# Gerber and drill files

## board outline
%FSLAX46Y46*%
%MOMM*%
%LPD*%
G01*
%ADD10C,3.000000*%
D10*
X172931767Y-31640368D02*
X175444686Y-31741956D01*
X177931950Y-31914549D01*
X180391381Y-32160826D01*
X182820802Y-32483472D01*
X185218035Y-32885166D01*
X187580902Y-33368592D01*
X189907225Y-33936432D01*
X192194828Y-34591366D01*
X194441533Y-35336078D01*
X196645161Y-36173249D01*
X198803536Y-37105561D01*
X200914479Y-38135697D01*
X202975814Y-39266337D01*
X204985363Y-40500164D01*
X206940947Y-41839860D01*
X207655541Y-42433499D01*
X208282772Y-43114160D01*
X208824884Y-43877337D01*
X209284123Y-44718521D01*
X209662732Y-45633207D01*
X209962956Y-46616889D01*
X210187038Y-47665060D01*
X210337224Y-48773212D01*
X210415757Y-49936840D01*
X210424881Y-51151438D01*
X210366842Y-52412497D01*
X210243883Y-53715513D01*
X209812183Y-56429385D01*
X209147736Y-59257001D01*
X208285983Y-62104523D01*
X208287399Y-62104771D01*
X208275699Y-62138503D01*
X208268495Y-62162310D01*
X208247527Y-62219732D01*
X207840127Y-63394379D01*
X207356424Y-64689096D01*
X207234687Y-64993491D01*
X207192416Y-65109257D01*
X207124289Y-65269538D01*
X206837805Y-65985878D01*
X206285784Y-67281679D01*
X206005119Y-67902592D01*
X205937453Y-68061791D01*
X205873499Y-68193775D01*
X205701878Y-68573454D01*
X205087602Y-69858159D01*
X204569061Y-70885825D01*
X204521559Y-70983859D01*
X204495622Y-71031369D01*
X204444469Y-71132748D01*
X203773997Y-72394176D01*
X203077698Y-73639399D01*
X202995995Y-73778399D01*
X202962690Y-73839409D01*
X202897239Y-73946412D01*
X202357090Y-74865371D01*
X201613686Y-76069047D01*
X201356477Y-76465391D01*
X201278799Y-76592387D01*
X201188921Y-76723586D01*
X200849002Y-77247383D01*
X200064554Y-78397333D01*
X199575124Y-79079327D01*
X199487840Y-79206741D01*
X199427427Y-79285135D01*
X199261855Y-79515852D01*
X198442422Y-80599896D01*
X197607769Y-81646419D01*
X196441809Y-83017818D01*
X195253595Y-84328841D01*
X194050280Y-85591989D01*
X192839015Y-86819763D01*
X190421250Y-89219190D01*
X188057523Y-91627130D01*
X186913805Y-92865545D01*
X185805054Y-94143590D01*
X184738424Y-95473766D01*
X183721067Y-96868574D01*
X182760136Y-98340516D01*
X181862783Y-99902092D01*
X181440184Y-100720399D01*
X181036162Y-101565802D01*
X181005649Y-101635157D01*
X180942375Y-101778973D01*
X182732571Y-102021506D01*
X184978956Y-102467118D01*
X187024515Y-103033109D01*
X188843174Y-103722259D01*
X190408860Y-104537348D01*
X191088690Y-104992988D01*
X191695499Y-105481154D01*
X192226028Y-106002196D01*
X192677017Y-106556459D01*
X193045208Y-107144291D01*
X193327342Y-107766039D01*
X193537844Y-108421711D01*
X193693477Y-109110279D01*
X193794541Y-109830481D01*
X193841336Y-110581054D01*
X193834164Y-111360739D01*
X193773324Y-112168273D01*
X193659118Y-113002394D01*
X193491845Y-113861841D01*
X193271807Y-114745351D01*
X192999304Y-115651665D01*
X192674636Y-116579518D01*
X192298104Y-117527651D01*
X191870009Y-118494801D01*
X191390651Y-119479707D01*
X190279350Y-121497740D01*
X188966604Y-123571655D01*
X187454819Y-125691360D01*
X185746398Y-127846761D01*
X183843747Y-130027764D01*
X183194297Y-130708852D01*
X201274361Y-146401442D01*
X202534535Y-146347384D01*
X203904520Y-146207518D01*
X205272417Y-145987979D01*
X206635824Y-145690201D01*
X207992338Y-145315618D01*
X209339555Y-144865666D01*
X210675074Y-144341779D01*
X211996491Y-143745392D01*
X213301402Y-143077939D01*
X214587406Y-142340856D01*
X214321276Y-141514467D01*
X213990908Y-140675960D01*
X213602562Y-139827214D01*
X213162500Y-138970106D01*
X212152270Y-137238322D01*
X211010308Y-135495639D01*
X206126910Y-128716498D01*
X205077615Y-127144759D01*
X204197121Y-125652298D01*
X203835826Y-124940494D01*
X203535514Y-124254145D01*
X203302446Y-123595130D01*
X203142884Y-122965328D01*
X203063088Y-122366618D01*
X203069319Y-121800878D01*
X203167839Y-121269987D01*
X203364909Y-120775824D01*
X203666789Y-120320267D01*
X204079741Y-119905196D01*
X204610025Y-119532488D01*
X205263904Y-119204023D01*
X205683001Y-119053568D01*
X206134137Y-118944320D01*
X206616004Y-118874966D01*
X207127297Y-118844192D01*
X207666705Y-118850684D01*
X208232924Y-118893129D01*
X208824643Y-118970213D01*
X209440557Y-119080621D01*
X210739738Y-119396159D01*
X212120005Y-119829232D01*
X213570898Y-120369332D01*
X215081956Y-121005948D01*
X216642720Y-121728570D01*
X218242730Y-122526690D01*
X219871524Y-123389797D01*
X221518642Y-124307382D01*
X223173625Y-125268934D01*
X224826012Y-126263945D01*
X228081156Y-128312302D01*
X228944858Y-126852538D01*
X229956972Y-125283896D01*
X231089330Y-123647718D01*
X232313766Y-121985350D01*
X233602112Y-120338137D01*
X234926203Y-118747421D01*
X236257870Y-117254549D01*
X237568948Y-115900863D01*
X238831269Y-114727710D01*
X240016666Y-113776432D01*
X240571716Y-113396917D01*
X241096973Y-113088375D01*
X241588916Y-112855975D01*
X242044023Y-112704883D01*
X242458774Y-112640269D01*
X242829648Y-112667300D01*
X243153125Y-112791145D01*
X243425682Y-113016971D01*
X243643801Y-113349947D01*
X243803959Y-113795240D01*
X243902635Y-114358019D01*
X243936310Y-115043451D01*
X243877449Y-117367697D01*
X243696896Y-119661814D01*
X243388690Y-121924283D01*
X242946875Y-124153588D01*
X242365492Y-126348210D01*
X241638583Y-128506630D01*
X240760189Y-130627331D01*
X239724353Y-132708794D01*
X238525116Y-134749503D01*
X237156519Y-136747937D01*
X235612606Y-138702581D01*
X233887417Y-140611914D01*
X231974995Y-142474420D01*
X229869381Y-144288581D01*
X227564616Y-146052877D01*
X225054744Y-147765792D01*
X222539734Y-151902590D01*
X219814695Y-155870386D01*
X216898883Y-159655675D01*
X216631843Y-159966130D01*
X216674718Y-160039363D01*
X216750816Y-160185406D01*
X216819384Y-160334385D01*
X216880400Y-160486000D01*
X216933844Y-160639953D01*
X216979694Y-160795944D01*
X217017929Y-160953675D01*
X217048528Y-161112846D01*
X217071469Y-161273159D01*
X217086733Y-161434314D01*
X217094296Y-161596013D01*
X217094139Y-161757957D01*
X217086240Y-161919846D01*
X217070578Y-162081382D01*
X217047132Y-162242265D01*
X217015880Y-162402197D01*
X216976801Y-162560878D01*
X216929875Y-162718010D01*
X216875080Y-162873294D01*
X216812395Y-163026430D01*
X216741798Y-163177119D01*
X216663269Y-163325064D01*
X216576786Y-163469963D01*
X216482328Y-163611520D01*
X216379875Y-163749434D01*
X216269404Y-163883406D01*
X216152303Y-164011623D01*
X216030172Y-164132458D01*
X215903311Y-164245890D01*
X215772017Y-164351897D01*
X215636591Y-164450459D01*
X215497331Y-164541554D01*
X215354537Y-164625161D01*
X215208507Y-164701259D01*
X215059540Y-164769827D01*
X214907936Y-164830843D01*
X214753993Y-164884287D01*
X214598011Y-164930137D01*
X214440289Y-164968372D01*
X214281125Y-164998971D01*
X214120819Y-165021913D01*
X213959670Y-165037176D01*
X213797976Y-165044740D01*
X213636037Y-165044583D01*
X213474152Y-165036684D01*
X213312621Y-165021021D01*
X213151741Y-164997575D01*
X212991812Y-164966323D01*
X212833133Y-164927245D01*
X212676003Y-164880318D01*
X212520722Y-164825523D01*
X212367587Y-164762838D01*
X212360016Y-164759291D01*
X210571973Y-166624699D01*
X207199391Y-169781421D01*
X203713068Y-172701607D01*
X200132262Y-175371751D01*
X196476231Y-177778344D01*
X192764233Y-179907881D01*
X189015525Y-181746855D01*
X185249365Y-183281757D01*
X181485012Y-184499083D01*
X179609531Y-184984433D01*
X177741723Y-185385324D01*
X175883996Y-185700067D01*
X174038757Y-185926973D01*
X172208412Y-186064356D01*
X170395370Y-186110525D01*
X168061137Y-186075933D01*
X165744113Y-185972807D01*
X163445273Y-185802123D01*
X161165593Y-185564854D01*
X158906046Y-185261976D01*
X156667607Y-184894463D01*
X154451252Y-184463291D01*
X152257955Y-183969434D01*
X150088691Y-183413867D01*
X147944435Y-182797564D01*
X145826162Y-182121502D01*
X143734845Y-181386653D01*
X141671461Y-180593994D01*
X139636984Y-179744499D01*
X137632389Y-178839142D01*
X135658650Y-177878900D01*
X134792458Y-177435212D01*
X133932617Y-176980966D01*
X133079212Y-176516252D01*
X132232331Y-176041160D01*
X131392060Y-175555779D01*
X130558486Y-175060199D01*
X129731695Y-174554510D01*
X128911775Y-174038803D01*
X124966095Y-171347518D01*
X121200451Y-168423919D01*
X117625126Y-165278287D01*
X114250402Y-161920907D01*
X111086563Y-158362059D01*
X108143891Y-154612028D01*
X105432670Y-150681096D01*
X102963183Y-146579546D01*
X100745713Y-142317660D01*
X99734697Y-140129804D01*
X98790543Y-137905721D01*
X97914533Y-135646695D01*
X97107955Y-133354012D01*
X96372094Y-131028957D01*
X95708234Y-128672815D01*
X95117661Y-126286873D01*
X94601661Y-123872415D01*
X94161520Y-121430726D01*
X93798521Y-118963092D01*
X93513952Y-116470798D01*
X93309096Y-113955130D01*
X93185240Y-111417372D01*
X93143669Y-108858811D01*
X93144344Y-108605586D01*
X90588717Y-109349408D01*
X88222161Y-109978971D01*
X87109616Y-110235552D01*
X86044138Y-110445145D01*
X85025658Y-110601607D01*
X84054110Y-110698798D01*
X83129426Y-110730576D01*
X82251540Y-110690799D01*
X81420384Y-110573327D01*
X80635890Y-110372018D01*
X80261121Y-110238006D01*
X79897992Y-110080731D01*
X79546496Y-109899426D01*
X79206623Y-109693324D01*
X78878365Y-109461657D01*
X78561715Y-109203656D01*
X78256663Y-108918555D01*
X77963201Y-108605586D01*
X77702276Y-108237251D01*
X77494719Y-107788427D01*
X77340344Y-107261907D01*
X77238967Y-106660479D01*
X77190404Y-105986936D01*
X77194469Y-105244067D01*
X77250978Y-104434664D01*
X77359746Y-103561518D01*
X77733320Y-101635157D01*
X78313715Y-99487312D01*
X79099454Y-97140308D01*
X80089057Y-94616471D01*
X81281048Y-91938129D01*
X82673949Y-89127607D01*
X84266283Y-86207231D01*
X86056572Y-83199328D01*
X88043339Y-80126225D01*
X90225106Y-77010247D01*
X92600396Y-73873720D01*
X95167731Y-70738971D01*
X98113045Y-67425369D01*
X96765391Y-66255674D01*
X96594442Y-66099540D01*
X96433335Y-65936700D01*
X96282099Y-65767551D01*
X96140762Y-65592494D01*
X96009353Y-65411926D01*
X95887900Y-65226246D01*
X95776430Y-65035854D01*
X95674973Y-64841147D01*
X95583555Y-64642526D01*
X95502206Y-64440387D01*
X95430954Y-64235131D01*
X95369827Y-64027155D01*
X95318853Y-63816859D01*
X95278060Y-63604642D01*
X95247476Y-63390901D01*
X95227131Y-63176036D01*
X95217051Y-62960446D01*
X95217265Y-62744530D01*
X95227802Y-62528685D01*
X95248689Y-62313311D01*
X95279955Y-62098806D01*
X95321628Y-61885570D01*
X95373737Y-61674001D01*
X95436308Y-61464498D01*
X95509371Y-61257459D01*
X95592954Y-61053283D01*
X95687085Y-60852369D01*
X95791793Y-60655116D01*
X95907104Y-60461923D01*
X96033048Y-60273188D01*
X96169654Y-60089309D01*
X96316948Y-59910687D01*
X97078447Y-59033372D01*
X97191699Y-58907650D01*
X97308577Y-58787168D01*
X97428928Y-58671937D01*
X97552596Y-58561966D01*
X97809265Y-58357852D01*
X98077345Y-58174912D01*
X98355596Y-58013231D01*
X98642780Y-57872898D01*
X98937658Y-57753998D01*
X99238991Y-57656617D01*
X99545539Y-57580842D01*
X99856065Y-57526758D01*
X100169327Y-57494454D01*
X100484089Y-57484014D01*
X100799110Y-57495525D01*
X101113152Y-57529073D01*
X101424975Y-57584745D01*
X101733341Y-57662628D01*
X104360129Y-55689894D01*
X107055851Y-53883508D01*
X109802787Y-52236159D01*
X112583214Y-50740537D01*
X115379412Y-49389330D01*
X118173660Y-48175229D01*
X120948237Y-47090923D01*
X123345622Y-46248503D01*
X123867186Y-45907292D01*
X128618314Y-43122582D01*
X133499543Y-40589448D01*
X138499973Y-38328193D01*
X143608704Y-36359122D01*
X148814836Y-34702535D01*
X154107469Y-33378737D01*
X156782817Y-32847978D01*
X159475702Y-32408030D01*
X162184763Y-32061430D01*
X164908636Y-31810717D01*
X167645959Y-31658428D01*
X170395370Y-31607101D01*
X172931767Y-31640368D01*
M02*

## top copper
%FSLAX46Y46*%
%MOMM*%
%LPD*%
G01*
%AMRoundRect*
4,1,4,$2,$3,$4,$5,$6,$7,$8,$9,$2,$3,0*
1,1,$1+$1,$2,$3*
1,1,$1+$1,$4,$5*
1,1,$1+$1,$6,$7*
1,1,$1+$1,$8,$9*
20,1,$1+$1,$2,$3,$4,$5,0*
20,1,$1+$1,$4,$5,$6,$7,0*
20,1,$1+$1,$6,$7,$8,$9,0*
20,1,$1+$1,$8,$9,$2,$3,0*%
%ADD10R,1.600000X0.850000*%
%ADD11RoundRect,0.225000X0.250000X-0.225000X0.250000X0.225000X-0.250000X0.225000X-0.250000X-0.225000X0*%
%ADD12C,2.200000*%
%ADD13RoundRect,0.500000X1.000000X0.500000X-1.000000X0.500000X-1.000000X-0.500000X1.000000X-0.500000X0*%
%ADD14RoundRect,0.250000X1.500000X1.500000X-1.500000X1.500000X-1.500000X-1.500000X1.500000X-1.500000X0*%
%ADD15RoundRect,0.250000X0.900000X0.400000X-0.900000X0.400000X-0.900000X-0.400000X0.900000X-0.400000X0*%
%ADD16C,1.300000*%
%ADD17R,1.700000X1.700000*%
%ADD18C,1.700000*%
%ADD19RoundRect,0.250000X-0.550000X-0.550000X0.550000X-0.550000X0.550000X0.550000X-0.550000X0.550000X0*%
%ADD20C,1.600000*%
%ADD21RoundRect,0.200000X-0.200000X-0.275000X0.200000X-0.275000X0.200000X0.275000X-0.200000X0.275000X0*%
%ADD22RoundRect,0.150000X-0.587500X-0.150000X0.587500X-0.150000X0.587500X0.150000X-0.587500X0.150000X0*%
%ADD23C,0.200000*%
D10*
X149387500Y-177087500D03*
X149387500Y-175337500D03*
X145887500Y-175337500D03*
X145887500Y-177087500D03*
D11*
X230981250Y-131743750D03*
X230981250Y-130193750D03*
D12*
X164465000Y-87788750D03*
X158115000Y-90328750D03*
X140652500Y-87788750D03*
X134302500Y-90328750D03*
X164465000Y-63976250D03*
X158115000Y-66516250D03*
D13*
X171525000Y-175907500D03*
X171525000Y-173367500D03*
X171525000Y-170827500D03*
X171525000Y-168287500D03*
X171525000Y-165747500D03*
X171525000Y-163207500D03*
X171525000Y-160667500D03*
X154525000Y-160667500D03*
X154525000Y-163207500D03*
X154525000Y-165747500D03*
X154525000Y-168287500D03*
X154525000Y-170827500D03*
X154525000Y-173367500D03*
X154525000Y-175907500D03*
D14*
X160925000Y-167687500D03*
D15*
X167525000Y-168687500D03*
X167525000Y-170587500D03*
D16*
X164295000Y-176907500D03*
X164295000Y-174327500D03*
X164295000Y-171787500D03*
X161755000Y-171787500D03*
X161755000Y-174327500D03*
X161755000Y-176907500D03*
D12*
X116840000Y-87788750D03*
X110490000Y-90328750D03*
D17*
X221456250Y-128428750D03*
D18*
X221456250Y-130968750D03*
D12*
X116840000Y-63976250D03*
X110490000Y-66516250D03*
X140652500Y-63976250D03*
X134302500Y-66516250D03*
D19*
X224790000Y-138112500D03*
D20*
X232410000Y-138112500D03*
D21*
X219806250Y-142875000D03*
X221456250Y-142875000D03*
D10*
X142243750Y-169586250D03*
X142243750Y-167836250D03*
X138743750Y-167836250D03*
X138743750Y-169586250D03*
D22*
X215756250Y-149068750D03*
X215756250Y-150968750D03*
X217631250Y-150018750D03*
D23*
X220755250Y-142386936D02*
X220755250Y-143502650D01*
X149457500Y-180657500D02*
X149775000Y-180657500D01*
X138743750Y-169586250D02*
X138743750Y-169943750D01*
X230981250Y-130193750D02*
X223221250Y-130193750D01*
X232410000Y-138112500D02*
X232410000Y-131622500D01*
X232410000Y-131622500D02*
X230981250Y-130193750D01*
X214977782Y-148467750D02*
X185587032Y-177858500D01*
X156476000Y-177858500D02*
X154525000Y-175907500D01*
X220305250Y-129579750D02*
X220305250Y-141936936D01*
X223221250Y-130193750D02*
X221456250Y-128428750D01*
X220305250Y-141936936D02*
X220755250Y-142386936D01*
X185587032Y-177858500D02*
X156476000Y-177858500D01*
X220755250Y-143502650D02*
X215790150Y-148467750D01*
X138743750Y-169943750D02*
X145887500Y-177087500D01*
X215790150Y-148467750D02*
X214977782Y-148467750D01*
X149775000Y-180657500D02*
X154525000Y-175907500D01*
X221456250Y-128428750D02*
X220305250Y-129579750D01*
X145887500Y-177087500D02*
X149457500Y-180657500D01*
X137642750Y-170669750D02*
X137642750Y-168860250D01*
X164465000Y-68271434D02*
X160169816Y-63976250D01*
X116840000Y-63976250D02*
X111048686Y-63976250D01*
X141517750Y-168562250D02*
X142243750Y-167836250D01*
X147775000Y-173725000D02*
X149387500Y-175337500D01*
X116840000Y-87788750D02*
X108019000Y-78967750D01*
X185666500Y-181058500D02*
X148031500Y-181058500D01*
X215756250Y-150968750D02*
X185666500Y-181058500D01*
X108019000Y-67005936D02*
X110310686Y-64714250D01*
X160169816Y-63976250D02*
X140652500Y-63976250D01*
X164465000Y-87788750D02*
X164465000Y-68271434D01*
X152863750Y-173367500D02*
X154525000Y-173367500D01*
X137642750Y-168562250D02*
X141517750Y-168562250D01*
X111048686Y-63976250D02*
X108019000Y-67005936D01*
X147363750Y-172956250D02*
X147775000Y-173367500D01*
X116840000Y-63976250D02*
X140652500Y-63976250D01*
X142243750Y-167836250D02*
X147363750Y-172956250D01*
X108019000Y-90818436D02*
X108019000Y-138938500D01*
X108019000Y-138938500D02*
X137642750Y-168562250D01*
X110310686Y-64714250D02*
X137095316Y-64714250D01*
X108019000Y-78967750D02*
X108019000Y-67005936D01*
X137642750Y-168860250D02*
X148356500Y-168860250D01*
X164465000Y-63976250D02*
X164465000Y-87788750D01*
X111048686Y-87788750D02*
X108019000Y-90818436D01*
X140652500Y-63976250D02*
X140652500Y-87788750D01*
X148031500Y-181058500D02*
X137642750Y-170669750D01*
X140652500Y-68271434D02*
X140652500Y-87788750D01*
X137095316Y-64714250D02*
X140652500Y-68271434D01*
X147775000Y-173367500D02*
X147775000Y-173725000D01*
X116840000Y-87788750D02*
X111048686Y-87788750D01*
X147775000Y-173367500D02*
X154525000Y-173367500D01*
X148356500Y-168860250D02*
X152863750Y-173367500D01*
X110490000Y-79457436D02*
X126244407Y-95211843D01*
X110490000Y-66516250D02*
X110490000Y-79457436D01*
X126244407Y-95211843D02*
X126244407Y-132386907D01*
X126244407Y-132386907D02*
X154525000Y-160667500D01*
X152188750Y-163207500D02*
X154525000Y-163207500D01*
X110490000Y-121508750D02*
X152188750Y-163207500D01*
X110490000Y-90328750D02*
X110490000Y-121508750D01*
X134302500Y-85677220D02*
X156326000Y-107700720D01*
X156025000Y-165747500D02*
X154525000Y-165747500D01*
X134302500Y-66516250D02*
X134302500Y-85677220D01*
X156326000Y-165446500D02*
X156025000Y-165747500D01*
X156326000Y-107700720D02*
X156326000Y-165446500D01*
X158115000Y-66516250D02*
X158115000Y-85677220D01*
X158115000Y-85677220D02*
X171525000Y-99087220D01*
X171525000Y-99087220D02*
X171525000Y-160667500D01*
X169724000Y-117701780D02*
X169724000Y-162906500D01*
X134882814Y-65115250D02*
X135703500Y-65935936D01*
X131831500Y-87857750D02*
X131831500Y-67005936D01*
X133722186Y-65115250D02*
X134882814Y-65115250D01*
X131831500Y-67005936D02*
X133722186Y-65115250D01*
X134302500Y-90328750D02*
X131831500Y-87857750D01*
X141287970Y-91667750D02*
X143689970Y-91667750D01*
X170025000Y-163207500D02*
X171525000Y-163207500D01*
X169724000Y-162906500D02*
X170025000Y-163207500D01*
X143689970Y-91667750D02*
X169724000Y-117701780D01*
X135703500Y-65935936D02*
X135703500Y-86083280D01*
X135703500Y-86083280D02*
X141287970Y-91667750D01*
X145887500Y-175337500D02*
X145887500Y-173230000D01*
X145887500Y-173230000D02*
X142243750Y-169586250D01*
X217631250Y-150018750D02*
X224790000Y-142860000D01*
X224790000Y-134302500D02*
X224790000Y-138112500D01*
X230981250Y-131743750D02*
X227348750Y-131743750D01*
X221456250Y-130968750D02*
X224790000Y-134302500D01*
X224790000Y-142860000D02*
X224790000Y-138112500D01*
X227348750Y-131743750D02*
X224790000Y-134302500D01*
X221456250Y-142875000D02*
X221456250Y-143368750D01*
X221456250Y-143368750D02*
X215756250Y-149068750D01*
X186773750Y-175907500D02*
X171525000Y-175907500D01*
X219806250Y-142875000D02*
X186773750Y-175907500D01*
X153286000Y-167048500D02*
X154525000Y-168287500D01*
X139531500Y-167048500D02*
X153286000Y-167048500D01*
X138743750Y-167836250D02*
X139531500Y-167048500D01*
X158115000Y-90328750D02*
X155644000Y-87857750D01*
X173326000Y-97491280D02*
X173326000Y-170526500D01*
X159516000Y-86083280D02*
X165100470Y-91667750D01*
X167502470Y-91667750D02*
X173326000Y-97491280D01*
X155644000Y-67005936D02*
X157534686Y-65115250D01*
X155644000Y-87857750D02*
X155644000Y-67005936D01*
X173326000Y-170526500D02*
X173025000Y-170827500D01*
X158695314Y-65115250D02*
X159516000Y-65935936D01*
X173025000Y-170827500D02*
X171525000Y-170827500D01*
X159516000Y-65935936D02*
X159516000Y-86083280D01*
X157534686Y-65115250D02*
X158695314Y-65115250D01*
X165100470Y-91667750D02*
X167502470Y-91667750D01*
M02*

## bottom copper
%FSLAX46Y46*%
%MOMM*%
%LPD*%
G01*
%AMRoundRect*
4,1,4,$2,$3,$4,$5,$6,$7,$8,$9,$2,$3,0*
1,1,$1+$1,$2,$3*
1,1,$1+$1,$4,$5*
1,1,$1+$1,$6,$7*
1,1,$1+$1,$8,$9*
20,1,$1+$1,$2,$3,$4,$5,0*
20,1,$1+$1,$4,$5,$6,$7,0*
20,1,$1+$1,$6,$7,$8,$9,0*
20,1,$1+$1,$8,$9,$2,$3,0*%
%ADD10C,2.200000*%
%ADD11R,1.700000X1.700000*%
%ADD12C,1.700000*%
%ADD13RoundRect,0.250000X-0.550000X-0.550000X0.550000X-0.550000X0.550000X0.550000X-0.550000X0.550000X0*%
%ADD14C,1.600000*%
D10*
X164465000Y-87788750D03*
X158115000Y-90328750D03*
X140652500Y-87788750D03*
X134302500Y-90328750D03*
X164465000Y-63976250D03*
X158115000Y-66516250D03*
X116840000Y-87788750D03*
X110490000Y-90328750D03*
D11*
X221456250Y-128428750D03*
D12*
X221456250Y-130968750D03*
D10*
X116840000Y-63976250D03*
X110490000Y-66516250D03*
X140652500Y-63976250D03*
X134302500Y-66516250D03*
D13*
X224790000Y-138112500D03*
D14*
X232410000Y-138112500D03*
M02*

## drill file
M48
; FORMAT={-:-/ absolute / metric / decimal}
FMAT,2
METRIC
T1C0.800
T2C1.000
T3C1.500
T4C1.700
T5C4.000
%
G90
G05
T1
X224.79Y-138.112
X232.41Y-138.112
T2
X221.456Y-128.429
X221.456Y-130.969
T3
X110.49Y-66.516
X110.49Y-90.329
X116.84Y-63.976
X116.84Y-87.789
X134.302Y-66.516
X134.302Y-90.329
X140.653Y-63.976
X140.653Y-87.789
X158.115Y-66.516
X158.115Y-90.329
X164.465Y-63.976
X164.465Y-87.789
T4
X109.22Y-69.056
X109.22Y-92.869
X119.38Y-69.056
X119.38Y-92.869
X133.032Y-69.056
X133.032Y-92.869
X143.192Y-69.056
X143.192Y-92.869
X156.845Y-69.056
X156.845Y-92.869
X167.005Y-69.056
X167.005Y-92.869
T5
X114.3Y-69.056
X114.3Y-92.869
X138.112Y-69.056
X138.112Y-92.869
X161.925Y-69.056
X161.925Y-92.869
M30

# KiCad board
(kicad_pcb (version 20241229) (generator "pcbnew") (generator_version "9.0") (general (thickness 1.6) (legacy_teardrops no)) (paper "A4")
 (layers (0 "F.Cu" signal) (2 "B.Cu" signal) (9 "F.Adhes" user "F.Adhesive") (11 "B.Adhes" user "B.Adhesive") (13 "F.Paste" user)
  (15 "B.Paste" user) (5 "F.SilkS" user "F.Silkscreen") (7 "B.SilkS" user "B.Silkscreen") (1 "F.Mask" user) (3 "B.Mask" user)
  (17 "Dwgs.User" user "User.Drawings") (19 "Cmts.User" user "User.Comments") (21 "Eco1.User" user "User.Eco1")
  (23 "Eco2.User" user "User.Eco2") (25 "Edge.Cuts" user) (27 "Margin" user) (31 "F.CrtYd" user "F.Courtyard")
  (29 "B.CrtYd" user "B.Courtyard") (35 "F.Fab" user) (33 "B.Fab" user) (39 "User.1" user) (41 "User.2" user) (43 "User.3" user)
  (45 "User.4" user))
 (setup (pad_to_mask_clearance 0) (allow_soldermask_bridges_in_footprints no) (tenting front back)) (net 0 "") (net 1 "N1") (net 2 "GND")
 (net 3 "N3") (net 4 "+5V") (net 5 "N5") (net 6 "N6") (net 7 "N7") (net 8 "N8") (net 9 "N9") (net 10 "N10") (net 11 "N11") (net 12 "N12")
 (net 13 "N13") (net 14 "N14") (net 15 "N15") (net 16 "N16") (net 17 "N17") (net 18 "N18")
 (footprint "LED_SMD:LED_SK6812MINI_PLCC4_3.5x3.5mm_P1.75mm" (layer "F.Cu") (at 147.6375 176.2125 180)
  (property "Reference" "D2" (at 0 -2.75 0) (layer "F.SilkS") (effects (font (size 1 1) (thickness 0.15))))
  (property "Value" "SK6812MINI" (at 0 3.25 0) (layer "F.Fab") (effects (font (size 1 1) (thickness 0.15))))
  (pad "1" smd rect (at -1.75 -0.875 180) (size 1.6 0.85) (layers "F.Cu" "F.Mask" "F.Paste") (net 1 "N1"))
  (pad "2" smd rect (at -1.75 0.875 180) (size 1.6 0.85) (layers "F.Cu" "F.Mask" "F.Paste") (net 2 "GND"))
  (pad "3" smd rect (at 1.75 0.875 180) (size 1.6 0.85) (layers "F.Cu" "F.Mask" "F.Paste") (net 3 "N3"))
  (pad "4" smd rect (at 1.75 -0.875 180) (size 1.6 0.85) (layers "F.Cu" "F.Mask" "F.Paste") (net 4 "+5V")))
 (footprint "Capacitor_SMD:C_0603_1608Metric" (layer "F.Cu") (at 230.98125 130.96875 90)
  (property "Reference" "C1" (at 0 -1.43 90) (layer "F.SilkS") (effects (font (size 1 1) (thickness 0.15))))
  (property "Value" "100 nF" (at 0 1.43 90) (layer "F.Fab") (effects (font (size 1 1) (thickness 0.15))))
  (pad "1" smd roundrect (at -0.775 0 90) (size 0.9 0.95) (layers "F.Cu" "F.Mask" "F.Paste") (roundrect_rratio 0.25) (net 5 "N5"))
  (pad "2" smd roundrect (at 0.775 0 90) (size 0.9 0.95) (layers "F.Cu" "F.Mask" "F.Paste") (roundrect_rratio 0.25) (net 4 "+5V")))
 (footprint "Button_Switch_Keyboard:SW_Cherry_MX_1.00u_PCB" (layer "F.Cu") (at 164.465 87.78875)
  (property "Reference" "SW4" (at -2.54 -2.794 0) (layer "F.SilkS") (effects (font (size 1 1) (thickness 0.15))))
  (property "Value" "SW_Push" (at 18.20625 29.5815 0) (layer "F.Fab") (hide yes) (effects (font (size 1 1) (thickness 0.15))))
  (pad "" np_thru_hole circle (at -7.62 5.08) (size 1.7 1.7) (drill 1.7) (layers "*.Cu" "*.Mask"))
  (pad "" np_thru_hole circle (at -2.54 5.08) (size 4 4) (drill 4) (layers "*.Cu" "*.Mask"))
  (pad "" np_thru_hole circle (at 2.54 5.08) (size 1.7 1.7) (drill 1.7) (layers "*.Cu" "*.Mask"))
  (pad "1" thru_hole circle (at 0 0) (size 2.2 2.2) (drill 1.5) (layers "*.Cu" "*.Mask") (remove_unused_layers no) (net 2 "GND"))
  (pad "2" thru_hole circle (at -6.35 2.54) (size 2.2 2.2) (drill 1.5) (layers "*.Cu" "*.Mask") (remove_unused_layers no) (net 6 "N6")))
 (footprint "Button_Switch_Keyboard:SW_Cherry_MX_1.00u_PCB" (layer "F.Cu") (at 140.6525 87.78875)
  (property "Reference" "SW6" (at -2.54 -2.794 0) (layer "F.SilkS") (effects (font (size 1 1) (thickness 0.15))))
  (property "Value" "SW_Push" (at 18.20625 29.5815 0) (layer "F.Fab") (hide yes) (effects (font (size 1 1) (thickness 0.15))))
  (pad "" np_thru_hole circle (at -7.62 5.08) (size 1.7 1.7) (drill 1.7) (layers "*.Cu" "*.Mask"))
  (pad "" np_thru_hole circle (at -2.54 5.08) (size 4 4) (drill 4) (layers "*.Cu" "*.Mask"))
  (pad "" np_thru_hole circle (at 2.54 5.08) (size 1.7 1.7) (drill 1.7) (layers "*.Cu" "*.Mask"))
  (pad "1" thru_hole circle (at 0 0) (size 2.2 2.2) (drill 1.5) (layers "*.Cu" "*.Mask") (remove_unused_layers no) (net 2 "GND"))
  (pad "2" thru_hole circle (at -6.35 2.54) (size 2.2 2.2) (drill 1.5) (layers "*.Cu" "*.Mask") (remove_unused_layers no) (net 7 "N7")))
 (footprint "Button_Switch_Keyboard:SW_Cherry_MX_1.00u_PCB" (layer "F.Cu") (at 164.465 63.97625)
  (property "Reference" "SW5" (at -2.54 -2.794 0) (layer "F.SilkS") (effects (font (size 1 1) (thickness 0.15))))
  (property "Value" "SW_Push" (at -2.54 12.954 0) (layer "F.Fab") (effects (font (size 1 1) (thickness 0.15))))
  (pad "" np_thru_hole circle (at -7.62 5.08) (size 1.7 1.7) (drill 1.7) (layers "*.Cu" "*.Mask"))
  (pad "" np_thru_hole circle (at -2.54 5.08) (size 4 4) (drill 4) (layers "*.Cu" "*.Mask"))
  (pad "" np_thru_hole circle (at 2.54 5.08) (size 1.7 1.7) (drill 1.7) (layers "*.Cu" "*.Mask"))
  (pad "1" thru_hole circle (at 0 0) (size 2.2 2.2) (drill 1.5) (layers "*.Cu" "*.Mask") (remove_unused_layers no) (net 2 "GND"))
  (pad "2" thru_hole circle (at -6.35 2.54) (size 2.2 2.2) (drill 1.5) (layers "*.Cu" "*.Mask") (remove_unused_layers no) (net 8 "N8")))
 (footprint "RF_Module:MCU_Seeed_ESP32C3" (layer "F.Cu") (at 163.025 168.2875 180)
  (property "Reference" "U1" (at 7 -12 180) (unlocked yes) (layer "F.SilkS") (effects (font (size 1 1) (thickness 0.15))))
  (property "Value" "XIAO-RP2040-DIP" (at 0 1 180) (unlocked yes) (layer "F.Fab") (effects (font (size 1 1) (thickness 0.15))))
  (pad "" smd roundrect (at 1.1 -0.4 180) (size 1.5 1.5) (layers "F.Paste") (roundrect_rratio 0.1666666667))
  (pad "" smd roundrect (at 1.1 1.6 180) (size 1.5 1.5) (layers "F.Paste") (roundrect_rratio 0.1666666667))
  (pad "" smd roundrect (at 3.1 -0.4 180) (size 1.5 1.5) (layers "F.Paste") (roundrect_rratio 0.1666666667))
  (pad "" smd roundrect (at 3.1 1.6 180) (size 1.5 1.5) (layers "F.Paste") (roundrect_rratio 0.1666666667))
  (pad "1" smd roundrect (at -8.5 -7.62 180) (size 3 2) (layers "F.Cu" "F.Mask" "F.Paste") (roundrect_rratio 0.25) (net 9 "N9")
   (thermal_bridge_angle 45))
  (pad "2" smd roundrect (at -8.5 -5.08 180) (size 3 2) (layers "F.Cu" "F.Mask" "F.Paste") (roundrect_rratio 0.25) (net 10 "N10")
   (thermal_bridge_angle 45))
  (pad "3" smd roundrect (at -8.5 -2.54 180) (size 3 2) (layers "F.Cu" "F.Mask" "F.Paste") (roundrect_rratio 0.25) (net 6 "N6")
   (thermal_bridge_angle 45))
  (pad "4" smd roundrect (at -8.5 0 180) (size 3 2) (layers "F.Cu" "F.Mask" "F.Paste") (roundrect_rratio 0.25) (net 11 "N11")
   (thermal_bridge_angle 45))
  (pad "5" smd roundrect (at -8.5 2.54 180) (size 3 2) (layers "F.Cu" "F.Mask" "F.Paste") (roundrect_rratio 0.25) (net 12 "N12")
   (thermal_bridge_angle 45))
  (pad "6" smd roundrect (at -8.5 5.08 180) (size 3 2) (layers "F.Cu" "F.Mask" "F.Paste") (roundrect_rratio 0.25) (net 7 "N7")
   (thermal_bridge_angle 45))
  (pad "7" smd roundrect (at -8.5 7.62 180) (size 3 2) (layers "F.Cu" "F.Mask" "F.Paste") (roundrect_rratio 0.25) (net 8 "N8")
   (thermal_bridge_angle 45))
  (pad "8" smd roundrect (at 8.5 7.62 180) (size 3 2) (layers "F.Cu" "F.Mask" "F.Paste") (roundrect_rratio 0.25) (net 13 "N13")
   (thermal_bridge_angle 45))
  (pad "9" smd roundrect (at 8.5 5.08 180) (size 3 2) (layers "F.Cu" "F.Mask" "F.Paste") (roundrect_rratio 0.25) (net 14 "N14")
   (thermal_bridge_angle 45))
  (pad "10" smd roundrect (at 8.5 2.54 180) (size 3 2) (layers "F.Cu" "F.Mask" "F.Paste") (roundrect_rratio 0.25) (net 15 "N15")
   (thermal_bridge_angle 45))
  (pad "11" smd roundrect (at 8.5 0 180) (size 3 2) (layers "F.Cu" "F.Mask" "F.Paste") (roundrect_rratio 0.25) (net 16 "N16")
   (thermal_bridge_angle 45))
  (pad "12" smd roundrect (at 8.5 -2.54 180) (size 3 2) (layers "F.Cu" "F.Mask" "F.Paste") (roundrect_rratio 0.25) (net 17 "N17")
   (thermal_bridge_angle 45))
  (pad "13" smd roundrect (at 8.5 -5.08 180) (size 3 2) (layers "F.Cu" "F.Mask" "F.Paste") (roundrect_rratio 0.25) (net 2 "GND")
   (thermal_bridge_angle 45))
  (pad "14" smd roundrect (at 8.5 -7.62 180) (size 3 2) (layers "F.Cu" "F.Mask" "F.Paste") (roundrect_rratio 0.25) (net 4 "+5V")
   (thermal_bridge_angle 45))
  (pad "15" smd roundrect (at 2.1 0.6 180) (size 3.5 3.5) (layers "F.Cu" "F.Mask") (roundrect_rratio 0.07142857143))
  (pad "16" smd roundrect (at -4.5 -0.4 180) (size 2.3 1.3) (layers "F.Cu" "F.Mask" "F.Paste") (roundrect_rratio 0.1923076923))
  (pad "17" smd roundrect (at -4.5 -2.3 180) (size 2.3 1.3) (layers "F.Cu" "F.Mask" "F.Paste") (roundrect_rratio 0.1923076923))
  (pad "18" smd circle (at -1.27 -8.62 180) (size 1.3 1.3) (layers "F.Cu" "F.Mask" "F.Paste"))
  (pad "19" smd circle (at -1.27 -6.04 180) (size 1.3 1.3) (layers "F.Cu" "F.Mask" "F.Paste"))
  (pad "20" smd circle (at -1.27 -3.5 180) (size 1.3 1.3) (layers "F.Cu" "F.Mask" "F.Paste"))
  (pad "21" smd circle (at 1.27 -3.5 180) (size 1.3 1.3) (layers "F.Cu" "F.Mask" "F.Paste"))
  (pad "22" smd circle (at 1.27 -6.04 180) (size 1.3 1.3) (layers "F.Cu" "F.Mask" "F.Paste"))
  (pad "23" smd circle (at 1.27 -8.62 180) (size 1.3 1.3) (layers "F.Cu" "F.Mask" "F.Paste")))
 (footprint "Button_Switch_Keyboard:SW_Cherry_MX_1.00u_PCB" (layer "F.Cu") (at 116.84 87.78875)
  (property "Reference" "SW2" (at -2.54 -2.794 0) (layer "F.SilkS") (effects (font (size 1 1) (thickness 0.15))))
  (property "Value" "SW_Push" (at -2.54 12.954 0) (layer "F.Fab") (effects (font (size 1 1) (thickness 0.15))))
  (pad "" np_thru_hole circle (at -7.62 5.08) (size 1.7 1.7) (drill 1.7) (layers "*.Cu" "*.Mask"))
  (pad "" np_thru_hole circle (at -2.54 5.08) (size 4 4) (drill 4) (layers "*.Cu" "*.Mask"))
  (pad "" np_thru_hole circle (at 2.54 5.08) (size 1.7 1.7) (drill 1.7) (layers "*.Cu" "*.Mask"))
  (pad "1" thru_hole circle (at 0 0) (size 2.2 2.2) (drill 1.5) (layers "*.Cu" "*.Mask") (remove_unused_layers no) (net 2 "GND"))
  (pad "2" thru_hole circle (at -6.35 2.54) (size 2.2 2.2) (drill 1.5) (layers "*.Cu" "*.Mask") (remove_unused_layers no) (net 14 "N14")))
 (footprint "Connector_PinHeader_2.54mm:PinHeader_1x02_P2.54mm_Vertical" (layer "F.Cu") (at 221.45625 128.42875)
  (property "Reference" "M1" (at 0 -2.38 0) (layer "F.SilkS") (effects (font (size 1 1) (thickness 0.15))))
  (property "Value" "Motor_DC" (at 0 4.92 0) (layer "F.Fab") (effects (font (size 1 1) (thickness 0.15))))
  (pad "1" thru_hole rect (at 0 0) (size 1.7 1.7) (drill 1) (layers "*.Cu" "*.Mask") (remove_unused_layers no) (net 4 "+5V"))
  (pad "2" thru_hole circle (at 0 2.54) (size 1.7 1.7) (drill 1) (layers "*.Cu" "*.Mask") (remove_unused_layers no) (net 5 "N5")))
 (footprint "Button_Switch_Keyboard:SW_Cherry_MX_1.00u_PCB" (layer "F.Cu") (at 116.84 63.97625)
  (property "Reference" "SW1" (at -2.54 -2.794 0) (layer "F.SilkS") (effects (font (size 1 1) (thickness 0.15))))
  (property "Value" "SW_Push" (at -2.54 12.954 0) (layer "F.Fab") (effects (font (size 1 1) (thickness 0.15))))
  (pad "" np_thru_hole circle (at -7.62 5.08) (size 1.7 1.7) (drill 1.7) (layers "*.Cu" "*.Mask"))
  (pad "" np_thru_hole circle (at -2.54 5.08) (size 4 4) (drill 4) (layers "*.Cu" "*.Mask"))
  (pad "" np_thru_hole circle (at 2.54 5.08) (size 1.7 1.7) (drill 1.7) (layers "*.Cu" "*.Mask"))
  (pad "1" thru_hole circle (at 0 0) (size 2.2 2.2) (drill 1.5) (layers "*.Cu" "*.Mask") (remove_unused_layers no) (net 2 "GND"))
  (pad "2" thru_hole circle (at -6.35 2.54) (size 2.2 2.2) (drill 1.5) (layers "*.Cu" "*.Mask") (remove_unused_layers no) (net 13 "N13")))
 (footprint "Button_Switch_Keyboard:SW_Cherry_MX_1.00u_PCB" (layer "F.Cu") (at 140.6525 63.97625)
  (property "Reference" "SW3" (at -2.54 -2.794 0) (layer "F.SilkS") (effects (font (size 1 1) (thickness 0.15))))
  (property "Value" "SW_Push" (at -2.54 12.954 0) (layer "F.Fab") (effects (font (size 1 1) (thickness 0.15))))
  (pad "" np_thru_hole circle (at -7.62 5.08) (size 1.7 1.7) (drill 1.7) (layers "*.Cu" "*.Mask"))
  (pad "" np_thru_hole circle (at -2.54 5.08) (size 4 4) (drill 4) (layers "*.Cu" "*.Mask"))
  (pad "" np_thru_hole circle (at 2.54 5.08) (size 1.7 1.7) (drill 1.7) (layers "*.Cu" "*.Mask"))
  (pad "1" thru_hole circle (at 0 0) (size 2.2 2.2) (drill 1.5) (layers "*.Cu" "*.Mask") (remove_unused_layers no) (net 2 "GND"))
  (pad "2" thru_hole circle (at -6.35 2.54) (size 2.2 2.2) (drill 1.5) (layers "*.Cu" "*.Mask") (remove_unused_layers no) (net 15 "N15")))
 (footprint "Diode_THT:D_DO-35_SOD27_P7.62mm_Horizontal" (layer "F.Cu") (at 224.79 138.1125)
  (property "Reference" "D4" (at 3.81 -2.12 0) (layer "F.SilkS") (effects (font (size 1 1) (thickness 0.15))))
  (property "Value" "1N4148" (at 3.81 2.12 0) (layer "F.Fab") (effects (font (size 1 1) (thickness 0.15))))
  (pad "1" thru_hole roundrect (at 0 0) (size 1.6 1.6) (drill 0.8) (layers "*.Cu" "*.Mask") (remove_unused_layers no)
   (roundrect_rratio 0.15625) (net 5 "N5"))
  (pad "2" thru_hole circle (at 7.62 0) (size 1.6 1.6) (drill 0.8) (layers "*.Cu" "*.Mask") (remove_unused_layers no) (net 4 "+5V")))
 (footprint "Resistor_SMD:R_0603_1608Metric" (layer "F.Cu") (at 220.63125 142.875)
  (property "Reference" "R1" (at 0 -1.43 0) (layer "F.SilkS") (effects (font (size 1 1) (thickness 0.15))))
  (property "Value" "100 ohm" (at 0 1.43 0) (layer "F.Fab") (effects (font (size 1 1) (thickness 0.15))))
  (pad "1" smd roundrect (at -0.825 0) (size 0.8 0.95) (layers "F.Cu" "F.Mask" "F.Paste") (roundrect_rratio 0.25) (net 9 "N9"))
  (pad "2" smd roundrect (at 0.825 0) (size 0.8 0.95) (layers "F.Cu" "F.Mask" "F.Paste") (roundrect_rratio 0.25) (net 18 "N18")))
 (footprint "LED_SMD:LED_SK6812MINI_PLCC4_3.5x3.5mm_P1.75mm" (layer "F.Cu") (at 140.49375 168.71125 180)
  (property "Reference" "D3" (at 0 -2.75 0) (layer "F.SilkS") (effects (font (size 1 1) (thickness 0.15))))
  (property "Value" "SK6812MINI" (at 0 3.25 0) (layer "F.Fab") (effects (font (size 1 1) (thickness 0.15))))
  (pad "1" smd rect (at -1.75 -0.875 180) (size 1.6 0.85) (layers "F.Cu" "F.Mask" "F.Paste") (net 3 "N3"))
  (pad "2" smd rect (at -1.75 0.875 180) (size 1.6 0.85) (layers "F.Cu" "F.Mask" "F.Paste") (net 2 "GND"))
  (pad "3" smd rect (at 1.75 0.875 180) (size 1.6 0.85) (layers "F.Cu" "F.Mask" "F.Paste") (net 16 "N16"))
  (pad "4" smd rect (at 1.75 -0.875 180) (size 1.6 0.85) (layers "F.Cu" "F.Mask" "F.Paste") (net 4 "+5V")))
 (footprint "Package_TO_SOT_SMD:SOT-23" (layer "F.Cu") (at 216.69375 150.01875)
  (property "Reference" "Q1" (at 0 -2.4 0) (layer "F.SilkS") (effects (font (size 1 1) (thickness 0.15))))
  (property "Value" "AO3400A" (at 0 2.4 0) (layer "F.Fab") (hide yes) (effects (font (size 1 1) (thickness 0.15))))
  (pad "1" smd roundrect (at -0.9375 -0.95) (size 1.475 0.6) (layers "F.Cu" "F.Mask" "F.Paste") (roundrect_rratio 0.25) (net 18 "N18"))
  (pad "2" smd roundrect (at -0.9375 0.95) (size 1.475 0.6) (layers "F.Cu" "F.Mask" "F.Paste") (roundrect_rratio 0.25) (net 2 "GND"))
  (pad "3" smd roundrect (at 0.9375 0) (size 1.475 0.6) (layers "F.Cu" "F.Mask" "F.Paste") (roundrect_rratio 0.25) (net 5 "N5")))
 (gr_poly
  (pts (xy 172.931767 31.640368) (xy 175.444686 31.741956) (xy 177.93195 31.914549) (xy 180.391381 32.160826) (xy 182.820802 32.483472)
   (xy 185.218035 32.885166) (xy 187.580902 33.368592) (xy 189.907225 33.936432) (xy 192.194828 34.591366) (xy 194.441533 35.336078)
   (xy 196.645161 36.173249) (xy 198.803536 37.105561) (xy 200.914479 38.135697) (xy 202.975814 39.266337) (xy 204.985363 40.500164)
   (xy 206.940947 41.83986) (xy 207.655541 42.433499) (xy 208.282772 43.11416) (xy 208.824884 43.877337) (xy 209.284123 44.718521)
   (xy 209.662732 45.633207) (xy 209.962956 46.616889) (xy 210.187038 47.66506) (xy 210.337224 48.773212) (xy 210.415757 49.93684)
   (xy 210.424881 51.151438) (xy 210.366842 52.412497) (xy 210.243883 53.715513) (xy 209.812183 56.429385) (xy 209.147736 59.257001)
   (xy 208.285983 62.104523) (xy 208.287399 62.104771) (xy 208.275699 62.138503) (xy 208.268495 62.16231) (xy 208.247527 62.219732)
   (xy 207.840127 63.394379) (xy 207.356424 64.689096) (xy 207.234687 64.993491) (xy 207.192416 65.109257) (xy 207.124289 65.269538)
   (xy 206.837805 65.985878) (xy 206.285784 67.281679) (xy 206.005119 67.902592) (xy 205.937453 68.061791) (xy 205.873499 68.193775)
   (xy 205.701878 68.573454) (xy 205.087602 69.858159) (xy 204.569061 70.885825) (xy 204.521559 70.983859) (xy 204.495622 71.031369)
   (xy 204.444469 71.132748) (xy 203.773997 72.394176) (xy 203.077698 73.639399) (xy 202.995995 73.778399) (xy 202.96269 73.839409)
   (xy 202.897239 73.946412) (xy 202.35709 74.865371) (xy 201.613686 76.069047) (xy 201.356477 76.465391) (xy 201.278799 76.592387)
   (xy 201.188921 76.723586) (xy 200.849002 77.247383) (xy 200.064554 78.397333) (xy 199.575124 79.079327) (xy 199.48784 79.206741)
   (xy 199.427427 79.285135) (xy 199.261855 79.515852) (xy 198.442422 80.599896) (xy 197.607769 81.646419) (xy 196.441809 83.017818)
   (xy 195.253595 84.328841) (xy 194.05028 85.591989) (xy 192.839015 86.819763) (xy 190.42125 89.21919) (xy 188.057523 91.62713)
   (xy 186.913805 92.865545) (xy 185.805054 94.14359) (xy 184.738424 95.473766) (xy 183.721067 96.868574) (xy 182.760136 98.340516)
   (xy 181.862783 99.902092) (xy 181.440184 100.720399) (xy 181.036162 101.565802) (xy 181.005649 101.635157) (xy 180.942375 101.778973)
   (xy 182.732571 102.021506) (xy 184.978956 102.467118) (xy 187.024515 103.033109) (xy 188.843174 103.722259) (xy 190.40886 104.537348)
   (xy 191.08869 104.992988) (xy 191.695499 105.481154) (xy 192.226028 106.002196) (xy 192.677017 106.556459) (xy 193.045208 107.144291)
   (xy 193.327342 107.766039) (xy 193.537844 108.421711) (xy 193.693477 109.110279) (xy 193.794541 109.830481) (xy 193.841336 110.581054)
   (xy 193.834164 111.360739) (xy 193.773324 112.168273) (xy 193.659118 113.002394) (xy 193.491845 113.861841) (xy 193.271807 114.745351)
   (xy 192.999304 115.651665) (xy 192.674636 116.579518) (xy 192.298104 117.527651) (xy 191.870009 118.494801) (xy 191.390651 119.479707)
   (xy 190.27935 121.49774) (xy 188.966604 123.571655) (xy 187.454819 125.69136) (xy 185.746398 127.846761) (xy 183.843747 130.027764)
   (xy 183.194297 130.708852) (xy 201.274361 146.401442) (xy 202.534535 146.347384) (xy 203.90452 146.207518) (xy 205.272417 145.987979)
   (xy 206.635824 145.690201) (xy 207.992338 145.315618) (xy 209.339555 144.865666) (xy 210.675074 144.341779) (xy 211.996491 143.745392)
   (xy 213.301402 143.077939) (xy 214.587406 142.340856) (xy 214.321276 141.514467) (xy 213.990908 140.67596) (xy 213.602562 139.827214)
   (xy 213.1625 138.970106) (xy 212.15227 137.238322) (xy 211.010308 135.495639) (xy 206.12691 128.716498) (xy 205.077615 127.144759)
   (xy 204.197121 125.652298) (xy 203.835826 124.940494) (xy 203.535514 124.254145) (xy 203.302446 123.59513) (xy 203.142884 122.965328)
   (xy 203.063088 122.366618) (xy 203.069319 121.800878) (xy 203.167839 121.269987) (xy 203.364909 120.775824) (xy 203.666789 120.320267)
   (xy 204.079741 119.905196) (xy 204.610025 119.532488) (xy 205.263904 119.204023) (xy 205.683001 119.053568) (xy 206.134137 118.94432)
   (xy 206.616004 118.874966) (xy 207.127297 118.844192) (xy 207.666705 118.850684) (xy 208.232924 118.893129) (xy 208.824643 118.970213)
   (xy 209.440557 119.080621) (xy 210.739738 119.396159) (xy 212.120005 119.829232) (xy 213.570898 120.369332) (xy 215.081956 121.005948)
   (xy 216.64272 121.72857) (xy 218.24273 122.52669) (xy 219.871524 123.389797) (xy 221.518642 124.307382) (xy 223.173625 125.268934)
   (xy 224.826012 126.263945) (xy 228.081156 128.312302) (xy 228.944858 126.852538) (xy 229.956972 125.283896) (xy 231.08933 123.647718)
   (xy 232.313766 121.98535) (xy 233.602112 120.338137) (xy 234.926203 118.747421) (xy 236.25787 117.254549) (xy 237.568948 115.900863)
   (xy 238.831269 114.72771) (xy 240.016666 113.776432) (xy 240.571716 113.396917) (xy 241.096973 113.088375) (xy 241.588916 112.855975)
   (xy 242.044023 112.704883) (xy 242.458774 112.640269) (xy 242.829648 112.6673) (xy 243.153125 112.791145) (xy 243.425682 113.016971)
   (xy 243.643801 113.349947) (xy 243.803959 113.79524) (xy 243.902635 114.358019) (xy 243.93631 115.043451) (xy 243.877449 117.367697)
   (xy 243.696896 119.661814) (xy 243.38869 121.924283) (xy 242.946875 124.153588) (xy 242.365492 126.34821) (xy 241.638583 128.50663)
   (xy 240.760189 130.627331) (xy 239.724353 132.708794) (xy 238.525116 134.749503) (xy 237.156519 136.747937) (xy 235.612606 138.702581)
   (xy 233.887417 140.611914) (xy 231.974995 142.47442) (xy 229.869381 144.288581) (xy 227.564616 146.052877) (xy 225.054744 147.765792)
   (xy 222.539734 151.90259) (xy 219.814695 155.870386) (xy 216.898883 159.655675) (xy 216.631843 159.96613) (xy 216.674718 160.039363)
   (xy 216.750816 160.185406) (xy 216.819384 160.334385) (xy 216.8804 160.486) (xy 216.933844 160.639953) (xy 216.979694 160.795944)
   (xy 217.017929 160.953675) (xy 217.048528 161.112846) (xy 217.071469 161.273159) (xy 217.086733 161.434314) (xy 217.094296 161.596013)
   (xy 217.094139 161.757957) (xy 217.08624 161.919846) (xy 217.070578 162.081382) (xy 217.047132 162.242265) (xy 217.01588 162.402197)
   (xy 216.976801 162.560878) (xy 216.929875 162.71801) (xy 216.87508 162.873294) (xy 216.812395 163.02643) (xy 216.741798 163.177119)
   (xy 216.663269 163.325064) (xy 216.576786 163.469963) (xy 216.482328 163.61152) (xy 216.379875 163.749434) (xy 216.269404 163.883406)
   (xy 216.152303 164.011623) (xy 216.030172 164.132458) (xy 215.903311 164.24589) (xy 215.772017 164.351897) (xy 215.636591 164.450459)
   (xy 215.497331 164.541554) (xy 215.354537 164.625161) (xy 215.208507 164.701259) (xy 215.05954 164.769827) (xy 214.907936 164.830843)
   (xy 214.753993 164.884287) (xy 214.598011 164.930137) (xy 214.440289 164.968372) (xy 214.281125 164.998971) (xy 214.120819 165.021913)
   (xy 213.95967 165.037176) (xy 213.797976 165.04474) (xy 213.636037 165.044583) (xy 213.474152 165.036684) (xy 213.312621 165.021021)
   (xy 213.151741 164.997575) (xy 212.991812 164.966323) (xy 212.833133 164.927245) (xy 212.676003 164.880318) (xy 212.520722 164.825523)
   (xy 212.367587 164.762838) (xy 212.360016 164.759291) (xy 210.571973 166.624699) (xy 207.199391 169.781421) (xy 203.713068 172.701607)
   (xy 200.132262 175.371751) (xy 196.476231 177.778344) (xy 192.764233 179.907881) (xy 189.015525 181.746855) (xy 185.249365 183.281757)
   (xy 181.485012 184.499083) (xy 179.609531 184.984433) (xy 177.741723 185.385324) (xy 175.883996 185.700067) (xy 174.038757 185.926973)
   (xy 172.208412 186.064356) (xy 170.39537 186.110525) (xy 168.061137 186.075933) (xy 165.744113 185.972807) (xy 163.445273 185.802123)
   (xy 161.165593 185.564854) (xy 158.906046 185.261976) (xy 156.667607 184.894463) (xy 154.451252 184.463291) (xy 152.257955 183.969434)
   (xy 150.088691 183.413867) (xy 147.944435 182.797564) (xy 145.826162 182.121502) (xy 143.734845 181.386653) (xy 141.671461 180.593994)
   (xy 139.636984 179.744499) (xy 137.632389 178.839142) (xy 135.65865 177.8789) (xy 134.792458 177.435212) (xy 133.932617 176.980966)
   (xy 133.079212 176.516252) (xy 132.232331 176.04116) (xy 131.39206 175.555779) (xy 130.558486 175.060199) (xy 129.731695 174.55451)
   (xy 128.911775 174.038803) (xy 124.966095 171.347518) (xy 121.200451 168.423919) (xy 117.625126 165.278287) (xy 114.250402 161.920907)
   (xy 111.086563 158.362059) (xy 108.143891 154.612028) (xy 105.43267 150.681096) (xy 102.963183 146.579546) (xy 100.745713 142.31766)
   (xy 99.734697 140.129804) (xy 98.790543 137.905721) (xy 97.914533 135.646695) (xy 97.107955 133.354012) (xy 96.372094 131.028957)
   (xy 95.708234 128.672815) (xy 95.117661 126.286873) (xy 94.601661 123.872415) (xy 94.16152 121.430726) (xy 93.798521 118.963092)
   (xy 93.513952 116.470798) (xy 93.309096 113.95513) (xy 93.18524 111.417372) (xy 93.143669 108.858811) (xy 93.144344 108.605586)
   (xy 90.588717 109.349408) (xy 88.222161 109.978971) (xy 87.109616 110.235552) (xy 86.044138 110.445145) (xy 85.025658 110.601607)
   (xy 84.05411 110.698798) (xy 83.129426 110.730576) (xy 82.25154 110.690799) (xy 81.420384 110.573327) (xy 80.63589 110.372018)
   (xy 80.261121 110.238006) (xy 79.897992 110.080731) (xy 79.546496 109.899426) (xy 79.206623 109.693324) (xy 78.878365 109.461657)
   (xy 78.561715 109.203656) (xy 78.256663 108.918555) (xy 77.963201 108.605586) (xy 77.702276 108.237251) (xy 77.494719 107.788427)
   (xy 77.340344 107.261907) (xy 77.238967 106.660479) (xy 77.190404 105.986936) (xy 77.194469 105.244067) (xy 77.250978 104.434664)
   (xy 77.359746 103.561518) (xy 77.73332 101.635157) (xy 78.313715 99.487312) (xy 79.099454 97.140308) (xy 80.089057 94.616471)
   (xy 81.281048 91.938129) (xy 82.673949 89.127607) (xy 84.266283 86.207231) (xy 86.056572 83.199328) (xy 88.043339 80.126225)
   (xy 90.225106 77.010247) (xy 92.600396 73.87372) (xy 95.167731 70.738971) (xy 98.113045 67.425369) (xy 96.765391 66.255674)
   (xy 96.594442 66.09954) (xy 96.433335 65.9367) (xy 96.282099 65.767551) (xy 96.140762 65.592494) (xy 96.009353 65.411926)
   (xy 95.8879 65.226246) (xy 95.77643 65.035854) (xy 95.674973 64.841147) (xy 95.583555 64.642526) (xy 95.502206 64.440387)
   (xy 95.430954 64.235131) (xy 95.369827 64.027155) (xy 95.318853 63.816859) (xy 95.27806 63.604642) (xy 95.247476 63.390901)
   (xy 95.227131 63.176036) (xy 95.217051 62.960446) (xy 95.217265 62.74453) (xy 95.227802 62.528685) (xy 95.248689 62.313311)
   (xy 95.279955 62.098806) (xy 95.321628 61.88557) (xy 95.373737 61.674001) (xy 95.436308 61.464498) (xy 95.509371 61.257459)
   (xy 95.592954 61.053283) (xy 95.687085 60.852369) (xy 95.791793 60.655116) (xy 95.907104 60.461923) (xy 96.033048 60.273188)
   (xy 96.169654 60.089309) (xy 96.316948 59.910687) (xy 97.078447 59.033372) (xy 97.191699 58.90765) (xy 97.308577 58.787168)
   (xy 97.428928 58.671937) (xy 97.552596 58.561966) (xy 97.809265 58.357852) (xy 98.077345 58.174912) (xy 98.355596 58.013231)
   (xy 98.64278 57.872898) (xy 98.937658 57.753998) (xy 99.238991 57.656617) (xy 99.545539 57.580842) (xy 99.856065 57.526758)
   (xy 100.169327 57.494454) (xy 100.484089 57.484014) (xy 100.79911 57.495525) (xy 101.113152 57.529073) (xy 101.424975 57.584745)
   (xy 101.733341 57.662628) (xy 104.360129 55.689894) (xy 107.055851 53.883508) (xy 109.802787 52.236159) (xy 112.583214 50.740537)
   (xy 115.379412 49.38933) (xy 118.17366 48.175229) (xy 120.948237 47.090923) (xy 123.345622 46.248503) (xy 123.867186 45.907292)
   (xy 128.618314 43.122582) (xy 133.499543 40.589448) (xy 138.499973 38.328193) (xy 143.608704 36.359122) (xy 148.814836 34.702535)
   (xy 154.107469 33.378737) (xy 156.782817 32.847978) (xy 159.475702 32.40803) (xy 162.184763 32.06143) (xy 164.908636 31.810717)
   (xy 167.645959 31.658428) (xy 170.39537 31.607101))
  (stroke (width 3) (type solid)) (fill no) (layer "Edge.Cuts"))
 (segment (start 220.75525 142.386936) (end 220.75525 143.50265) (width 0.2) (layer "F.Cu") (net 4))
 (segment (start 149.4575 180.6575) (end 149.775 180.6575) (width 0.2) (layer "F.Cu") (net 4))
 (segment (start 138.74375 169.58625) (end 138.74375 169.94375) (width 0.2) (layer "F.Cu") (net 4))
 (segment (start 230.98125 130.19375) (end 223.22125 130.19375) (width 0.2) (layer "F.Cu") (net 4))
 (segment (start 232.41 138.1125) (end 232.41 131.6225) (width 0.2) (layer "F.Cu") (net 4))
 (segment (start 232.41 131.6225) (end 230.98125 130.19375) (width 0.2) (layer "F.Cu") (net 4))
 (segment (start 214.977782 148.46775) (end 185.587032 177.8585) (width 0.2) (layer "F.Cu") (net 4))
 (segment (start 156.476 177.8585) (end 154.525 175.9075) (width 0.2) (layer "F.Cu") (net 4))
 (segment (start 220.30525 129.57975) (end 220.30525 141.936936) (width 0.2) (layer "F.Cu") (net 4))
 (segment (start 223.22125 130.19375) (end 221.45625 128.42875) (width 0.2) (layer "F.Cu") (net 4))
 (segment (start 220.30525 141.936936) (end 220.75525 142.386936) (width 0.2) (layer "F.Cu") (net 4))
 (segment (start 185.587032 177.8585) (end 156.476 177.8585) (width 0.2) (layer "F.Cu") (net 4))
 (segment (start 220.75525 143.50265) (end 215.79015 148.46775) (width 0.2) (layer "F.Cu") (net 4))
 (segment (start 138.74375 169.94375) (end 145.8875 177.0875) (width 0.2) (layer "F.Cu") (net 4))
 (segment (start 215.79015 148.46775) (end 214.977782 148.46775) (width 0.2) (layer "F.Cu") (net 4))
 (segment (start 149.775 180.6575) (end 154.525 175.9075) (width 0.2) (layer "F.Cu") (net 4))
 (segment (start 221.45625 128.42875) (end 220.30525 129.57975) (width 0.2) (layer "F.Cu") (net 4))
 (segment (start 145.8875 177.0875) (end 149.4575 180.6575) (width 0.2) (layer "F.Cu") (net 4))
 (segment (start 137.64275 170.66975) (end 137.64275 168.86025) (width 0.2) (layer "F.Cu") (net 2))
 (segment (start 164.465 68.271434) (end 160.169816 63.97625) (width 0.2) (layer "F.Cu") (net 2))
 (segment (start 116.84 63.97625) (end 111.048686 63.97625) (width 0.2) (layer "F.Cu") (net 2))
 (segment (start 141.51775 168.56225) (end 142.24375 167.83625) (width 0.2) (layer "F.Cu") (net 2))
 (segment (start 147.775 173.725) (end 149.3875 175.3375) (width 0.2) (layer "F.Cu") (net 2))
 (segment (start 116.84 87.78875) (end 108.019 78.96775) (width 0.2) (layer "F.Cu") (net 2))
 (segment (start 185.6665 181.0585) (end 148.0315 181.0585) (width 0.2) (layer "F.Cu") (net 2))
 (segment (start 215.75625 150.96875) (end 185.6665 181.0585) (width 0.2) (layer "F.Cu") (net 2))
 (segment (start 108.019 67.005936) (end 110.310686 64.71425) (width 0.2) (layer "F.Cu") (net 2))
 (segment (start 160.169816 63.97625) (end 140.6525 63.97625) (width 0.2) (layer "F.Cu") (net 2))
 (segment (start 164.465 87.78875) (end 164.465 68.271434) (width 0.2) (layer "F.Cu") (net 2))
 (segment (start 152.86375 173.3675) (end 154.525 173.3675) (width 0.2) (layer "F.Cu") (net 2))
 (segment (start 137.64275 168.56225) (end 141.51775 168.56225) (width 0.2) (layer "F.Cu") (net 2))
 (segment (start 111.048686 63.97625) (end 108.019 67.005936) (width 0.2) (layer "F.Cu") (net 2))
 (segment (start 147.36375 172.95625) (end 147.775 173.3675) (width 0.2) (layer "F.Cu") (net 2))
 (segment (start 116.84 63.97625) (end 140.6525 63.97625) (width 0.2) (layer "F.Cu") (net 2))
 (segment (start 142.24375 167.83625) (end 147.36375 172.95625) (width 0.2) (layer "F.Cu") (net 2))
 (segment (start 108.019 90.818436) (end 108.019 138.9385) (width 0.2) (layer "F.Cu") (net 2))
 (segment (start 108.019 138.9385) (end 137.64275 168.56225) (width 0.2) (layer "F.Cu") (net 2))
 (segment (start 110.310686 64.71425) (end 137.095316 64.71425) (width 0.2) (layer "F.Cu") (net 2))
 (segment (start 108.019 78.96775) (end 108.019 67.005936) (width 0.2) (layer "F.Cu") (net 2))
 (segment (start 137.64275 168.86025) (end 148.3565 168.86025) (width 0.2) (layer "F.Cu") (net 2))
 (segment (start 164.465 63.97625) (end 164.465 87.78875) (width 0.2) (layer "F.Cu") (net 2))
 (segment (start 111.048686 87.78875) (end 108.019 90.818436) (width 0.2) (layer "F.Cu") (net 2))
 (segment (start 140.6525 63.97625) (end 140.6525 87.78875) (width 0.2) (layer "F.Cu") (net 2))
 (segment (start 148.0315 181.0585) (end 137.64275 170.66975) (width 0.2) (layer "F.Cu") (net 2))
 (segment (start 140.6525 68.271434) (end 140.6525 87.78875) (width 0.2) (layer "F.Cu") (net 2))
 (segment (start 137.095316 64.71425) (end 140.6525 68.271434) (width 0.2) (layer "F.Cu") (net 2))
 (segment (start 147.775 173.3675) (end 147.775 173.725) (width 0.2) (layer "F.Cu") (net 2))
 (segment (start 116.84 87.78875) (end 111.048686 87.78875) (width 0.2) (layer "F.Cu") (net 2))
 (segment (start 147.775 173.3675) (end 154.525 173.3675) (width 0.2) (layer "F.Cu") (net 2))
 (segment (start 148.3565 168.86025) (end 152.86375 173.3675) (width 0.2) (layer "F.Cu") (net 2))
 (segment (start 110.49 79.457436) (end 126.244407 95.211843) (width 0.2) (layer "F.Cu") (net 13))
 (segment (start 110.49 66.51625) (end 110.49 79.457436) (width 0.2) (layer "F.Cu") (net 13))
 (segment (start 126.244407 95.211843) (end 126.244407 132.386907) (width 0.2) (layer "F.Cu") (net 13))
 (segment (start 126.244407 132.386907) (end 154.525 160.6675) (width 0.2) (layer "F.Cu") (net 13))
 (segment (start 152.18875 163.2075) (end 154.525 163.2075) (width 0.2) (layer "F.Cu") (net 14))
 (segment (start 110.49 121.50875) (end 152.18875 163.2075) (width 0.2) (layer "F.Cu") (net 14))
 (segment (start 110.49 90.32875) (end 110.49 121.50875) (width 0.2) (layer "F.Cu") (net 14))
 (segment (start 134.3025 85.67722) (end 156.326 107.70072) (width 0.2) (layer "F.Cu") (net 15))
 (segment (start 156.025 165.7475) (end 154.525 165.7475) (width 0.2) (layer "F.Cu") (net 15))
 (segment (start 134.3025 66.51625) (end 134.3025 85.67722) (width 0.2) (layer "F.Cu") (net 15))
 (segment (start 156.326 165.4465) (end 156.025 165.7475) (width 0.2) (layer "F.Cu") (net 15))
 (segment (start 156.326 107.70072) (end 156.326 165.4465) (width 0.2) (layer "F.Cu") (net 15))
 (segment (start 158.115 66.51625) (end 158.115 85.67722) (width 0.2) (layer "F.Cu") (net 8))
 (segment (start 158.115 85.67722) (end 171.525 99.08722) (width 0.2) (layer "F.Cu") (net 8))
 (segment (start 171.525 99.08722) (end 171.525 160.6675) (width 0.2) (layer "F.Cu") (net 8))
 (segment (start 169.724 117.70178) (end 169.724 162.9065) (width 0.2) (layer "F.Cu") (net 7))
 (segment (start 134.882814 65.11525) (end 135.7035 65.935936) (width 0.2) (layer "F.Cu") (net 7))
 (segment (start 131.8315 87.85775) (end 131.8315 67.005936) (width 0.2) (layer "F.Cu") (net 7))
 (segment (start 133.722186 65.11525) (end 134.882814 65.11525) (width 0.2) (layer "F.Cu") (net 7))
 (segment (start 131.8315 67.005936) (end 133.722186 65.11525) (width 0.2) (layer "F.Cu") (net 7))
 (segment (start 134.3025 90.32875) (end 131.8315 87.85775) (width 0.2) (layer "F.Cu") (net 7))
 (segment (start 141.28797 91.66775) (end 143.68997 91.66775) (width 0.2) (layer "F.Cu") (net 7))
 (segment (start 170.025 163.2075) (end 171.525 163.2075) (width 0.2) (layer "F.Cu") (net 7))
 (segment (start 169.724 162.9065) (end 170.025 163.2075) (width 0.2) (layer "F.Cu") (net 7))
 (segment (start 143.68997 91.66775) (end 169.724 117.70178) (width 0.2) (layer "F.Cu") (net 7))
 (segment (start 135.7035 65.935936) (end 135.7035 86.08328) (width 0.2) (layer "F.Cu") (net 7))
 (segment (start 135.7035 86.08328) (end 141.28797 91.66775) (width 0.2) (layer "F.Cu") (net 7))
 (segment (start 145.8875 175.3375) (end 145.8875 173.23) (width 0.2) (layer "F.Cu") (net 3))
 (segment (start 145.8875 173.23) (end 142.24375 169.58625) (width 0.2) (layer "F.Cu") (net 3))
 (segment (start 217.63125 150.01875) (end 224.79 142.86) (width 0.2) (layer "F.Cu") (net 5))
 (segment (start 224.79 134.3025) (end 224.79 138.1125) (width 0.2) (layer "F.Cu") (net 5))
 (segment (start 230.98125 131.74375) (end 227.34875 131.74375) (width 0.2) (layer "F.Cu") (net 5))
 (segment (start 221.45625 130.96875) (end 224.79 134.3025) (width 0.2) (layer "F.Cu") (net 5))
 (segment (start 224.79 142.86) (end 224.79 138.1125) (width 0.2) (layer "F.Cu") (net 5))
 (segment (start 227.34875 131.74375) (end 224.79 134.3025) (width 0.2) (layer "F.Cu") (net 5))
 (segment (start 221.45625 142.875) (end 221.45625 143.36875) (width 0.2) (layer "F.Cu") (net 18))
 (segment (start 221.45625 143.36875) (end 215.75625 149.06875) (width 0.2) (layer "F.Cu") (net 18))
 (segment (start 186.77375 175.9075) (end 171.525 175.9075) (width 0.2) (layer "F.Cu") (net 9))
 (segment (start 219.80625 142.875) (end 186.77375 175.9075) (width 0.2) (layer "F.Cu") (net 9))
 (segment (start 153.286 167.0485) (end 154.525 168.2875) (width 0.2) (layer "F.Cu") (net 16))
 (segment (start 139.5315 167.0485) (end 153.286 167.0485) (width 0.2) (layer "F.Cu") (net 16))
 (segment (start 138.74375 167.83625) (end 139.5315 167.0485) (width 0.2) (layer "F.Cu") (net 16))
 (segment (start 158.115 90.32875) (end 155.644 87.85775) (width 0.2) (layer "F.Cu") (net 6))
 (segment (start 173.326 97.49128) (end 173.326 170.5265) (width 0.2) (layer "F.Cu") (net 6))
 (segment (start 159.516 86.08328) (end 165.10047 91.66775) (width 0.2) (layer "F.Cu") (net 6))
 (segment (start 167.50247 91.66775) (end 173.326 97.49128) (width 0.2) (layer "F.Cu") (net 6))
 (segment (start 155.644 67.005936) (end 157.534686 65.11525) (width 0.2) (layer "F.Cu") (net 6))
 (segment (start 155.644 87.85775) (end 155.644 67.005936) (width 0.2) (layer "F.Cu") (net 6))
 (segment (start 173.326 170.5265) (end 173.025 170.8275) (width 0.2) (layer "F.Cu") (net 6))
 (segment (start 158.695314 65.11525) (end 159.516 65.935936) (width 0.2) (layer "F.Cu") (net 6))
 (segment (start 173.025 170.8275) (end 171.525 170.8275) (width 0.2) (layer "F.Cu") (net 6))
 (segment (start 159.516 65.935936) (end 159.516 86.08328) (width 0.2) (layer "F.Cu") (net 6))
 (segment (start 157.534686 65.11525) (end 158.695314 65.11525) (width 0.2) (layer "F.Cu") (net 6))
 (segment (start 165.10047 91.66775) (end 167.50247 91.66775) (width 0.2) (layer "F.Cu") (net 6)))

